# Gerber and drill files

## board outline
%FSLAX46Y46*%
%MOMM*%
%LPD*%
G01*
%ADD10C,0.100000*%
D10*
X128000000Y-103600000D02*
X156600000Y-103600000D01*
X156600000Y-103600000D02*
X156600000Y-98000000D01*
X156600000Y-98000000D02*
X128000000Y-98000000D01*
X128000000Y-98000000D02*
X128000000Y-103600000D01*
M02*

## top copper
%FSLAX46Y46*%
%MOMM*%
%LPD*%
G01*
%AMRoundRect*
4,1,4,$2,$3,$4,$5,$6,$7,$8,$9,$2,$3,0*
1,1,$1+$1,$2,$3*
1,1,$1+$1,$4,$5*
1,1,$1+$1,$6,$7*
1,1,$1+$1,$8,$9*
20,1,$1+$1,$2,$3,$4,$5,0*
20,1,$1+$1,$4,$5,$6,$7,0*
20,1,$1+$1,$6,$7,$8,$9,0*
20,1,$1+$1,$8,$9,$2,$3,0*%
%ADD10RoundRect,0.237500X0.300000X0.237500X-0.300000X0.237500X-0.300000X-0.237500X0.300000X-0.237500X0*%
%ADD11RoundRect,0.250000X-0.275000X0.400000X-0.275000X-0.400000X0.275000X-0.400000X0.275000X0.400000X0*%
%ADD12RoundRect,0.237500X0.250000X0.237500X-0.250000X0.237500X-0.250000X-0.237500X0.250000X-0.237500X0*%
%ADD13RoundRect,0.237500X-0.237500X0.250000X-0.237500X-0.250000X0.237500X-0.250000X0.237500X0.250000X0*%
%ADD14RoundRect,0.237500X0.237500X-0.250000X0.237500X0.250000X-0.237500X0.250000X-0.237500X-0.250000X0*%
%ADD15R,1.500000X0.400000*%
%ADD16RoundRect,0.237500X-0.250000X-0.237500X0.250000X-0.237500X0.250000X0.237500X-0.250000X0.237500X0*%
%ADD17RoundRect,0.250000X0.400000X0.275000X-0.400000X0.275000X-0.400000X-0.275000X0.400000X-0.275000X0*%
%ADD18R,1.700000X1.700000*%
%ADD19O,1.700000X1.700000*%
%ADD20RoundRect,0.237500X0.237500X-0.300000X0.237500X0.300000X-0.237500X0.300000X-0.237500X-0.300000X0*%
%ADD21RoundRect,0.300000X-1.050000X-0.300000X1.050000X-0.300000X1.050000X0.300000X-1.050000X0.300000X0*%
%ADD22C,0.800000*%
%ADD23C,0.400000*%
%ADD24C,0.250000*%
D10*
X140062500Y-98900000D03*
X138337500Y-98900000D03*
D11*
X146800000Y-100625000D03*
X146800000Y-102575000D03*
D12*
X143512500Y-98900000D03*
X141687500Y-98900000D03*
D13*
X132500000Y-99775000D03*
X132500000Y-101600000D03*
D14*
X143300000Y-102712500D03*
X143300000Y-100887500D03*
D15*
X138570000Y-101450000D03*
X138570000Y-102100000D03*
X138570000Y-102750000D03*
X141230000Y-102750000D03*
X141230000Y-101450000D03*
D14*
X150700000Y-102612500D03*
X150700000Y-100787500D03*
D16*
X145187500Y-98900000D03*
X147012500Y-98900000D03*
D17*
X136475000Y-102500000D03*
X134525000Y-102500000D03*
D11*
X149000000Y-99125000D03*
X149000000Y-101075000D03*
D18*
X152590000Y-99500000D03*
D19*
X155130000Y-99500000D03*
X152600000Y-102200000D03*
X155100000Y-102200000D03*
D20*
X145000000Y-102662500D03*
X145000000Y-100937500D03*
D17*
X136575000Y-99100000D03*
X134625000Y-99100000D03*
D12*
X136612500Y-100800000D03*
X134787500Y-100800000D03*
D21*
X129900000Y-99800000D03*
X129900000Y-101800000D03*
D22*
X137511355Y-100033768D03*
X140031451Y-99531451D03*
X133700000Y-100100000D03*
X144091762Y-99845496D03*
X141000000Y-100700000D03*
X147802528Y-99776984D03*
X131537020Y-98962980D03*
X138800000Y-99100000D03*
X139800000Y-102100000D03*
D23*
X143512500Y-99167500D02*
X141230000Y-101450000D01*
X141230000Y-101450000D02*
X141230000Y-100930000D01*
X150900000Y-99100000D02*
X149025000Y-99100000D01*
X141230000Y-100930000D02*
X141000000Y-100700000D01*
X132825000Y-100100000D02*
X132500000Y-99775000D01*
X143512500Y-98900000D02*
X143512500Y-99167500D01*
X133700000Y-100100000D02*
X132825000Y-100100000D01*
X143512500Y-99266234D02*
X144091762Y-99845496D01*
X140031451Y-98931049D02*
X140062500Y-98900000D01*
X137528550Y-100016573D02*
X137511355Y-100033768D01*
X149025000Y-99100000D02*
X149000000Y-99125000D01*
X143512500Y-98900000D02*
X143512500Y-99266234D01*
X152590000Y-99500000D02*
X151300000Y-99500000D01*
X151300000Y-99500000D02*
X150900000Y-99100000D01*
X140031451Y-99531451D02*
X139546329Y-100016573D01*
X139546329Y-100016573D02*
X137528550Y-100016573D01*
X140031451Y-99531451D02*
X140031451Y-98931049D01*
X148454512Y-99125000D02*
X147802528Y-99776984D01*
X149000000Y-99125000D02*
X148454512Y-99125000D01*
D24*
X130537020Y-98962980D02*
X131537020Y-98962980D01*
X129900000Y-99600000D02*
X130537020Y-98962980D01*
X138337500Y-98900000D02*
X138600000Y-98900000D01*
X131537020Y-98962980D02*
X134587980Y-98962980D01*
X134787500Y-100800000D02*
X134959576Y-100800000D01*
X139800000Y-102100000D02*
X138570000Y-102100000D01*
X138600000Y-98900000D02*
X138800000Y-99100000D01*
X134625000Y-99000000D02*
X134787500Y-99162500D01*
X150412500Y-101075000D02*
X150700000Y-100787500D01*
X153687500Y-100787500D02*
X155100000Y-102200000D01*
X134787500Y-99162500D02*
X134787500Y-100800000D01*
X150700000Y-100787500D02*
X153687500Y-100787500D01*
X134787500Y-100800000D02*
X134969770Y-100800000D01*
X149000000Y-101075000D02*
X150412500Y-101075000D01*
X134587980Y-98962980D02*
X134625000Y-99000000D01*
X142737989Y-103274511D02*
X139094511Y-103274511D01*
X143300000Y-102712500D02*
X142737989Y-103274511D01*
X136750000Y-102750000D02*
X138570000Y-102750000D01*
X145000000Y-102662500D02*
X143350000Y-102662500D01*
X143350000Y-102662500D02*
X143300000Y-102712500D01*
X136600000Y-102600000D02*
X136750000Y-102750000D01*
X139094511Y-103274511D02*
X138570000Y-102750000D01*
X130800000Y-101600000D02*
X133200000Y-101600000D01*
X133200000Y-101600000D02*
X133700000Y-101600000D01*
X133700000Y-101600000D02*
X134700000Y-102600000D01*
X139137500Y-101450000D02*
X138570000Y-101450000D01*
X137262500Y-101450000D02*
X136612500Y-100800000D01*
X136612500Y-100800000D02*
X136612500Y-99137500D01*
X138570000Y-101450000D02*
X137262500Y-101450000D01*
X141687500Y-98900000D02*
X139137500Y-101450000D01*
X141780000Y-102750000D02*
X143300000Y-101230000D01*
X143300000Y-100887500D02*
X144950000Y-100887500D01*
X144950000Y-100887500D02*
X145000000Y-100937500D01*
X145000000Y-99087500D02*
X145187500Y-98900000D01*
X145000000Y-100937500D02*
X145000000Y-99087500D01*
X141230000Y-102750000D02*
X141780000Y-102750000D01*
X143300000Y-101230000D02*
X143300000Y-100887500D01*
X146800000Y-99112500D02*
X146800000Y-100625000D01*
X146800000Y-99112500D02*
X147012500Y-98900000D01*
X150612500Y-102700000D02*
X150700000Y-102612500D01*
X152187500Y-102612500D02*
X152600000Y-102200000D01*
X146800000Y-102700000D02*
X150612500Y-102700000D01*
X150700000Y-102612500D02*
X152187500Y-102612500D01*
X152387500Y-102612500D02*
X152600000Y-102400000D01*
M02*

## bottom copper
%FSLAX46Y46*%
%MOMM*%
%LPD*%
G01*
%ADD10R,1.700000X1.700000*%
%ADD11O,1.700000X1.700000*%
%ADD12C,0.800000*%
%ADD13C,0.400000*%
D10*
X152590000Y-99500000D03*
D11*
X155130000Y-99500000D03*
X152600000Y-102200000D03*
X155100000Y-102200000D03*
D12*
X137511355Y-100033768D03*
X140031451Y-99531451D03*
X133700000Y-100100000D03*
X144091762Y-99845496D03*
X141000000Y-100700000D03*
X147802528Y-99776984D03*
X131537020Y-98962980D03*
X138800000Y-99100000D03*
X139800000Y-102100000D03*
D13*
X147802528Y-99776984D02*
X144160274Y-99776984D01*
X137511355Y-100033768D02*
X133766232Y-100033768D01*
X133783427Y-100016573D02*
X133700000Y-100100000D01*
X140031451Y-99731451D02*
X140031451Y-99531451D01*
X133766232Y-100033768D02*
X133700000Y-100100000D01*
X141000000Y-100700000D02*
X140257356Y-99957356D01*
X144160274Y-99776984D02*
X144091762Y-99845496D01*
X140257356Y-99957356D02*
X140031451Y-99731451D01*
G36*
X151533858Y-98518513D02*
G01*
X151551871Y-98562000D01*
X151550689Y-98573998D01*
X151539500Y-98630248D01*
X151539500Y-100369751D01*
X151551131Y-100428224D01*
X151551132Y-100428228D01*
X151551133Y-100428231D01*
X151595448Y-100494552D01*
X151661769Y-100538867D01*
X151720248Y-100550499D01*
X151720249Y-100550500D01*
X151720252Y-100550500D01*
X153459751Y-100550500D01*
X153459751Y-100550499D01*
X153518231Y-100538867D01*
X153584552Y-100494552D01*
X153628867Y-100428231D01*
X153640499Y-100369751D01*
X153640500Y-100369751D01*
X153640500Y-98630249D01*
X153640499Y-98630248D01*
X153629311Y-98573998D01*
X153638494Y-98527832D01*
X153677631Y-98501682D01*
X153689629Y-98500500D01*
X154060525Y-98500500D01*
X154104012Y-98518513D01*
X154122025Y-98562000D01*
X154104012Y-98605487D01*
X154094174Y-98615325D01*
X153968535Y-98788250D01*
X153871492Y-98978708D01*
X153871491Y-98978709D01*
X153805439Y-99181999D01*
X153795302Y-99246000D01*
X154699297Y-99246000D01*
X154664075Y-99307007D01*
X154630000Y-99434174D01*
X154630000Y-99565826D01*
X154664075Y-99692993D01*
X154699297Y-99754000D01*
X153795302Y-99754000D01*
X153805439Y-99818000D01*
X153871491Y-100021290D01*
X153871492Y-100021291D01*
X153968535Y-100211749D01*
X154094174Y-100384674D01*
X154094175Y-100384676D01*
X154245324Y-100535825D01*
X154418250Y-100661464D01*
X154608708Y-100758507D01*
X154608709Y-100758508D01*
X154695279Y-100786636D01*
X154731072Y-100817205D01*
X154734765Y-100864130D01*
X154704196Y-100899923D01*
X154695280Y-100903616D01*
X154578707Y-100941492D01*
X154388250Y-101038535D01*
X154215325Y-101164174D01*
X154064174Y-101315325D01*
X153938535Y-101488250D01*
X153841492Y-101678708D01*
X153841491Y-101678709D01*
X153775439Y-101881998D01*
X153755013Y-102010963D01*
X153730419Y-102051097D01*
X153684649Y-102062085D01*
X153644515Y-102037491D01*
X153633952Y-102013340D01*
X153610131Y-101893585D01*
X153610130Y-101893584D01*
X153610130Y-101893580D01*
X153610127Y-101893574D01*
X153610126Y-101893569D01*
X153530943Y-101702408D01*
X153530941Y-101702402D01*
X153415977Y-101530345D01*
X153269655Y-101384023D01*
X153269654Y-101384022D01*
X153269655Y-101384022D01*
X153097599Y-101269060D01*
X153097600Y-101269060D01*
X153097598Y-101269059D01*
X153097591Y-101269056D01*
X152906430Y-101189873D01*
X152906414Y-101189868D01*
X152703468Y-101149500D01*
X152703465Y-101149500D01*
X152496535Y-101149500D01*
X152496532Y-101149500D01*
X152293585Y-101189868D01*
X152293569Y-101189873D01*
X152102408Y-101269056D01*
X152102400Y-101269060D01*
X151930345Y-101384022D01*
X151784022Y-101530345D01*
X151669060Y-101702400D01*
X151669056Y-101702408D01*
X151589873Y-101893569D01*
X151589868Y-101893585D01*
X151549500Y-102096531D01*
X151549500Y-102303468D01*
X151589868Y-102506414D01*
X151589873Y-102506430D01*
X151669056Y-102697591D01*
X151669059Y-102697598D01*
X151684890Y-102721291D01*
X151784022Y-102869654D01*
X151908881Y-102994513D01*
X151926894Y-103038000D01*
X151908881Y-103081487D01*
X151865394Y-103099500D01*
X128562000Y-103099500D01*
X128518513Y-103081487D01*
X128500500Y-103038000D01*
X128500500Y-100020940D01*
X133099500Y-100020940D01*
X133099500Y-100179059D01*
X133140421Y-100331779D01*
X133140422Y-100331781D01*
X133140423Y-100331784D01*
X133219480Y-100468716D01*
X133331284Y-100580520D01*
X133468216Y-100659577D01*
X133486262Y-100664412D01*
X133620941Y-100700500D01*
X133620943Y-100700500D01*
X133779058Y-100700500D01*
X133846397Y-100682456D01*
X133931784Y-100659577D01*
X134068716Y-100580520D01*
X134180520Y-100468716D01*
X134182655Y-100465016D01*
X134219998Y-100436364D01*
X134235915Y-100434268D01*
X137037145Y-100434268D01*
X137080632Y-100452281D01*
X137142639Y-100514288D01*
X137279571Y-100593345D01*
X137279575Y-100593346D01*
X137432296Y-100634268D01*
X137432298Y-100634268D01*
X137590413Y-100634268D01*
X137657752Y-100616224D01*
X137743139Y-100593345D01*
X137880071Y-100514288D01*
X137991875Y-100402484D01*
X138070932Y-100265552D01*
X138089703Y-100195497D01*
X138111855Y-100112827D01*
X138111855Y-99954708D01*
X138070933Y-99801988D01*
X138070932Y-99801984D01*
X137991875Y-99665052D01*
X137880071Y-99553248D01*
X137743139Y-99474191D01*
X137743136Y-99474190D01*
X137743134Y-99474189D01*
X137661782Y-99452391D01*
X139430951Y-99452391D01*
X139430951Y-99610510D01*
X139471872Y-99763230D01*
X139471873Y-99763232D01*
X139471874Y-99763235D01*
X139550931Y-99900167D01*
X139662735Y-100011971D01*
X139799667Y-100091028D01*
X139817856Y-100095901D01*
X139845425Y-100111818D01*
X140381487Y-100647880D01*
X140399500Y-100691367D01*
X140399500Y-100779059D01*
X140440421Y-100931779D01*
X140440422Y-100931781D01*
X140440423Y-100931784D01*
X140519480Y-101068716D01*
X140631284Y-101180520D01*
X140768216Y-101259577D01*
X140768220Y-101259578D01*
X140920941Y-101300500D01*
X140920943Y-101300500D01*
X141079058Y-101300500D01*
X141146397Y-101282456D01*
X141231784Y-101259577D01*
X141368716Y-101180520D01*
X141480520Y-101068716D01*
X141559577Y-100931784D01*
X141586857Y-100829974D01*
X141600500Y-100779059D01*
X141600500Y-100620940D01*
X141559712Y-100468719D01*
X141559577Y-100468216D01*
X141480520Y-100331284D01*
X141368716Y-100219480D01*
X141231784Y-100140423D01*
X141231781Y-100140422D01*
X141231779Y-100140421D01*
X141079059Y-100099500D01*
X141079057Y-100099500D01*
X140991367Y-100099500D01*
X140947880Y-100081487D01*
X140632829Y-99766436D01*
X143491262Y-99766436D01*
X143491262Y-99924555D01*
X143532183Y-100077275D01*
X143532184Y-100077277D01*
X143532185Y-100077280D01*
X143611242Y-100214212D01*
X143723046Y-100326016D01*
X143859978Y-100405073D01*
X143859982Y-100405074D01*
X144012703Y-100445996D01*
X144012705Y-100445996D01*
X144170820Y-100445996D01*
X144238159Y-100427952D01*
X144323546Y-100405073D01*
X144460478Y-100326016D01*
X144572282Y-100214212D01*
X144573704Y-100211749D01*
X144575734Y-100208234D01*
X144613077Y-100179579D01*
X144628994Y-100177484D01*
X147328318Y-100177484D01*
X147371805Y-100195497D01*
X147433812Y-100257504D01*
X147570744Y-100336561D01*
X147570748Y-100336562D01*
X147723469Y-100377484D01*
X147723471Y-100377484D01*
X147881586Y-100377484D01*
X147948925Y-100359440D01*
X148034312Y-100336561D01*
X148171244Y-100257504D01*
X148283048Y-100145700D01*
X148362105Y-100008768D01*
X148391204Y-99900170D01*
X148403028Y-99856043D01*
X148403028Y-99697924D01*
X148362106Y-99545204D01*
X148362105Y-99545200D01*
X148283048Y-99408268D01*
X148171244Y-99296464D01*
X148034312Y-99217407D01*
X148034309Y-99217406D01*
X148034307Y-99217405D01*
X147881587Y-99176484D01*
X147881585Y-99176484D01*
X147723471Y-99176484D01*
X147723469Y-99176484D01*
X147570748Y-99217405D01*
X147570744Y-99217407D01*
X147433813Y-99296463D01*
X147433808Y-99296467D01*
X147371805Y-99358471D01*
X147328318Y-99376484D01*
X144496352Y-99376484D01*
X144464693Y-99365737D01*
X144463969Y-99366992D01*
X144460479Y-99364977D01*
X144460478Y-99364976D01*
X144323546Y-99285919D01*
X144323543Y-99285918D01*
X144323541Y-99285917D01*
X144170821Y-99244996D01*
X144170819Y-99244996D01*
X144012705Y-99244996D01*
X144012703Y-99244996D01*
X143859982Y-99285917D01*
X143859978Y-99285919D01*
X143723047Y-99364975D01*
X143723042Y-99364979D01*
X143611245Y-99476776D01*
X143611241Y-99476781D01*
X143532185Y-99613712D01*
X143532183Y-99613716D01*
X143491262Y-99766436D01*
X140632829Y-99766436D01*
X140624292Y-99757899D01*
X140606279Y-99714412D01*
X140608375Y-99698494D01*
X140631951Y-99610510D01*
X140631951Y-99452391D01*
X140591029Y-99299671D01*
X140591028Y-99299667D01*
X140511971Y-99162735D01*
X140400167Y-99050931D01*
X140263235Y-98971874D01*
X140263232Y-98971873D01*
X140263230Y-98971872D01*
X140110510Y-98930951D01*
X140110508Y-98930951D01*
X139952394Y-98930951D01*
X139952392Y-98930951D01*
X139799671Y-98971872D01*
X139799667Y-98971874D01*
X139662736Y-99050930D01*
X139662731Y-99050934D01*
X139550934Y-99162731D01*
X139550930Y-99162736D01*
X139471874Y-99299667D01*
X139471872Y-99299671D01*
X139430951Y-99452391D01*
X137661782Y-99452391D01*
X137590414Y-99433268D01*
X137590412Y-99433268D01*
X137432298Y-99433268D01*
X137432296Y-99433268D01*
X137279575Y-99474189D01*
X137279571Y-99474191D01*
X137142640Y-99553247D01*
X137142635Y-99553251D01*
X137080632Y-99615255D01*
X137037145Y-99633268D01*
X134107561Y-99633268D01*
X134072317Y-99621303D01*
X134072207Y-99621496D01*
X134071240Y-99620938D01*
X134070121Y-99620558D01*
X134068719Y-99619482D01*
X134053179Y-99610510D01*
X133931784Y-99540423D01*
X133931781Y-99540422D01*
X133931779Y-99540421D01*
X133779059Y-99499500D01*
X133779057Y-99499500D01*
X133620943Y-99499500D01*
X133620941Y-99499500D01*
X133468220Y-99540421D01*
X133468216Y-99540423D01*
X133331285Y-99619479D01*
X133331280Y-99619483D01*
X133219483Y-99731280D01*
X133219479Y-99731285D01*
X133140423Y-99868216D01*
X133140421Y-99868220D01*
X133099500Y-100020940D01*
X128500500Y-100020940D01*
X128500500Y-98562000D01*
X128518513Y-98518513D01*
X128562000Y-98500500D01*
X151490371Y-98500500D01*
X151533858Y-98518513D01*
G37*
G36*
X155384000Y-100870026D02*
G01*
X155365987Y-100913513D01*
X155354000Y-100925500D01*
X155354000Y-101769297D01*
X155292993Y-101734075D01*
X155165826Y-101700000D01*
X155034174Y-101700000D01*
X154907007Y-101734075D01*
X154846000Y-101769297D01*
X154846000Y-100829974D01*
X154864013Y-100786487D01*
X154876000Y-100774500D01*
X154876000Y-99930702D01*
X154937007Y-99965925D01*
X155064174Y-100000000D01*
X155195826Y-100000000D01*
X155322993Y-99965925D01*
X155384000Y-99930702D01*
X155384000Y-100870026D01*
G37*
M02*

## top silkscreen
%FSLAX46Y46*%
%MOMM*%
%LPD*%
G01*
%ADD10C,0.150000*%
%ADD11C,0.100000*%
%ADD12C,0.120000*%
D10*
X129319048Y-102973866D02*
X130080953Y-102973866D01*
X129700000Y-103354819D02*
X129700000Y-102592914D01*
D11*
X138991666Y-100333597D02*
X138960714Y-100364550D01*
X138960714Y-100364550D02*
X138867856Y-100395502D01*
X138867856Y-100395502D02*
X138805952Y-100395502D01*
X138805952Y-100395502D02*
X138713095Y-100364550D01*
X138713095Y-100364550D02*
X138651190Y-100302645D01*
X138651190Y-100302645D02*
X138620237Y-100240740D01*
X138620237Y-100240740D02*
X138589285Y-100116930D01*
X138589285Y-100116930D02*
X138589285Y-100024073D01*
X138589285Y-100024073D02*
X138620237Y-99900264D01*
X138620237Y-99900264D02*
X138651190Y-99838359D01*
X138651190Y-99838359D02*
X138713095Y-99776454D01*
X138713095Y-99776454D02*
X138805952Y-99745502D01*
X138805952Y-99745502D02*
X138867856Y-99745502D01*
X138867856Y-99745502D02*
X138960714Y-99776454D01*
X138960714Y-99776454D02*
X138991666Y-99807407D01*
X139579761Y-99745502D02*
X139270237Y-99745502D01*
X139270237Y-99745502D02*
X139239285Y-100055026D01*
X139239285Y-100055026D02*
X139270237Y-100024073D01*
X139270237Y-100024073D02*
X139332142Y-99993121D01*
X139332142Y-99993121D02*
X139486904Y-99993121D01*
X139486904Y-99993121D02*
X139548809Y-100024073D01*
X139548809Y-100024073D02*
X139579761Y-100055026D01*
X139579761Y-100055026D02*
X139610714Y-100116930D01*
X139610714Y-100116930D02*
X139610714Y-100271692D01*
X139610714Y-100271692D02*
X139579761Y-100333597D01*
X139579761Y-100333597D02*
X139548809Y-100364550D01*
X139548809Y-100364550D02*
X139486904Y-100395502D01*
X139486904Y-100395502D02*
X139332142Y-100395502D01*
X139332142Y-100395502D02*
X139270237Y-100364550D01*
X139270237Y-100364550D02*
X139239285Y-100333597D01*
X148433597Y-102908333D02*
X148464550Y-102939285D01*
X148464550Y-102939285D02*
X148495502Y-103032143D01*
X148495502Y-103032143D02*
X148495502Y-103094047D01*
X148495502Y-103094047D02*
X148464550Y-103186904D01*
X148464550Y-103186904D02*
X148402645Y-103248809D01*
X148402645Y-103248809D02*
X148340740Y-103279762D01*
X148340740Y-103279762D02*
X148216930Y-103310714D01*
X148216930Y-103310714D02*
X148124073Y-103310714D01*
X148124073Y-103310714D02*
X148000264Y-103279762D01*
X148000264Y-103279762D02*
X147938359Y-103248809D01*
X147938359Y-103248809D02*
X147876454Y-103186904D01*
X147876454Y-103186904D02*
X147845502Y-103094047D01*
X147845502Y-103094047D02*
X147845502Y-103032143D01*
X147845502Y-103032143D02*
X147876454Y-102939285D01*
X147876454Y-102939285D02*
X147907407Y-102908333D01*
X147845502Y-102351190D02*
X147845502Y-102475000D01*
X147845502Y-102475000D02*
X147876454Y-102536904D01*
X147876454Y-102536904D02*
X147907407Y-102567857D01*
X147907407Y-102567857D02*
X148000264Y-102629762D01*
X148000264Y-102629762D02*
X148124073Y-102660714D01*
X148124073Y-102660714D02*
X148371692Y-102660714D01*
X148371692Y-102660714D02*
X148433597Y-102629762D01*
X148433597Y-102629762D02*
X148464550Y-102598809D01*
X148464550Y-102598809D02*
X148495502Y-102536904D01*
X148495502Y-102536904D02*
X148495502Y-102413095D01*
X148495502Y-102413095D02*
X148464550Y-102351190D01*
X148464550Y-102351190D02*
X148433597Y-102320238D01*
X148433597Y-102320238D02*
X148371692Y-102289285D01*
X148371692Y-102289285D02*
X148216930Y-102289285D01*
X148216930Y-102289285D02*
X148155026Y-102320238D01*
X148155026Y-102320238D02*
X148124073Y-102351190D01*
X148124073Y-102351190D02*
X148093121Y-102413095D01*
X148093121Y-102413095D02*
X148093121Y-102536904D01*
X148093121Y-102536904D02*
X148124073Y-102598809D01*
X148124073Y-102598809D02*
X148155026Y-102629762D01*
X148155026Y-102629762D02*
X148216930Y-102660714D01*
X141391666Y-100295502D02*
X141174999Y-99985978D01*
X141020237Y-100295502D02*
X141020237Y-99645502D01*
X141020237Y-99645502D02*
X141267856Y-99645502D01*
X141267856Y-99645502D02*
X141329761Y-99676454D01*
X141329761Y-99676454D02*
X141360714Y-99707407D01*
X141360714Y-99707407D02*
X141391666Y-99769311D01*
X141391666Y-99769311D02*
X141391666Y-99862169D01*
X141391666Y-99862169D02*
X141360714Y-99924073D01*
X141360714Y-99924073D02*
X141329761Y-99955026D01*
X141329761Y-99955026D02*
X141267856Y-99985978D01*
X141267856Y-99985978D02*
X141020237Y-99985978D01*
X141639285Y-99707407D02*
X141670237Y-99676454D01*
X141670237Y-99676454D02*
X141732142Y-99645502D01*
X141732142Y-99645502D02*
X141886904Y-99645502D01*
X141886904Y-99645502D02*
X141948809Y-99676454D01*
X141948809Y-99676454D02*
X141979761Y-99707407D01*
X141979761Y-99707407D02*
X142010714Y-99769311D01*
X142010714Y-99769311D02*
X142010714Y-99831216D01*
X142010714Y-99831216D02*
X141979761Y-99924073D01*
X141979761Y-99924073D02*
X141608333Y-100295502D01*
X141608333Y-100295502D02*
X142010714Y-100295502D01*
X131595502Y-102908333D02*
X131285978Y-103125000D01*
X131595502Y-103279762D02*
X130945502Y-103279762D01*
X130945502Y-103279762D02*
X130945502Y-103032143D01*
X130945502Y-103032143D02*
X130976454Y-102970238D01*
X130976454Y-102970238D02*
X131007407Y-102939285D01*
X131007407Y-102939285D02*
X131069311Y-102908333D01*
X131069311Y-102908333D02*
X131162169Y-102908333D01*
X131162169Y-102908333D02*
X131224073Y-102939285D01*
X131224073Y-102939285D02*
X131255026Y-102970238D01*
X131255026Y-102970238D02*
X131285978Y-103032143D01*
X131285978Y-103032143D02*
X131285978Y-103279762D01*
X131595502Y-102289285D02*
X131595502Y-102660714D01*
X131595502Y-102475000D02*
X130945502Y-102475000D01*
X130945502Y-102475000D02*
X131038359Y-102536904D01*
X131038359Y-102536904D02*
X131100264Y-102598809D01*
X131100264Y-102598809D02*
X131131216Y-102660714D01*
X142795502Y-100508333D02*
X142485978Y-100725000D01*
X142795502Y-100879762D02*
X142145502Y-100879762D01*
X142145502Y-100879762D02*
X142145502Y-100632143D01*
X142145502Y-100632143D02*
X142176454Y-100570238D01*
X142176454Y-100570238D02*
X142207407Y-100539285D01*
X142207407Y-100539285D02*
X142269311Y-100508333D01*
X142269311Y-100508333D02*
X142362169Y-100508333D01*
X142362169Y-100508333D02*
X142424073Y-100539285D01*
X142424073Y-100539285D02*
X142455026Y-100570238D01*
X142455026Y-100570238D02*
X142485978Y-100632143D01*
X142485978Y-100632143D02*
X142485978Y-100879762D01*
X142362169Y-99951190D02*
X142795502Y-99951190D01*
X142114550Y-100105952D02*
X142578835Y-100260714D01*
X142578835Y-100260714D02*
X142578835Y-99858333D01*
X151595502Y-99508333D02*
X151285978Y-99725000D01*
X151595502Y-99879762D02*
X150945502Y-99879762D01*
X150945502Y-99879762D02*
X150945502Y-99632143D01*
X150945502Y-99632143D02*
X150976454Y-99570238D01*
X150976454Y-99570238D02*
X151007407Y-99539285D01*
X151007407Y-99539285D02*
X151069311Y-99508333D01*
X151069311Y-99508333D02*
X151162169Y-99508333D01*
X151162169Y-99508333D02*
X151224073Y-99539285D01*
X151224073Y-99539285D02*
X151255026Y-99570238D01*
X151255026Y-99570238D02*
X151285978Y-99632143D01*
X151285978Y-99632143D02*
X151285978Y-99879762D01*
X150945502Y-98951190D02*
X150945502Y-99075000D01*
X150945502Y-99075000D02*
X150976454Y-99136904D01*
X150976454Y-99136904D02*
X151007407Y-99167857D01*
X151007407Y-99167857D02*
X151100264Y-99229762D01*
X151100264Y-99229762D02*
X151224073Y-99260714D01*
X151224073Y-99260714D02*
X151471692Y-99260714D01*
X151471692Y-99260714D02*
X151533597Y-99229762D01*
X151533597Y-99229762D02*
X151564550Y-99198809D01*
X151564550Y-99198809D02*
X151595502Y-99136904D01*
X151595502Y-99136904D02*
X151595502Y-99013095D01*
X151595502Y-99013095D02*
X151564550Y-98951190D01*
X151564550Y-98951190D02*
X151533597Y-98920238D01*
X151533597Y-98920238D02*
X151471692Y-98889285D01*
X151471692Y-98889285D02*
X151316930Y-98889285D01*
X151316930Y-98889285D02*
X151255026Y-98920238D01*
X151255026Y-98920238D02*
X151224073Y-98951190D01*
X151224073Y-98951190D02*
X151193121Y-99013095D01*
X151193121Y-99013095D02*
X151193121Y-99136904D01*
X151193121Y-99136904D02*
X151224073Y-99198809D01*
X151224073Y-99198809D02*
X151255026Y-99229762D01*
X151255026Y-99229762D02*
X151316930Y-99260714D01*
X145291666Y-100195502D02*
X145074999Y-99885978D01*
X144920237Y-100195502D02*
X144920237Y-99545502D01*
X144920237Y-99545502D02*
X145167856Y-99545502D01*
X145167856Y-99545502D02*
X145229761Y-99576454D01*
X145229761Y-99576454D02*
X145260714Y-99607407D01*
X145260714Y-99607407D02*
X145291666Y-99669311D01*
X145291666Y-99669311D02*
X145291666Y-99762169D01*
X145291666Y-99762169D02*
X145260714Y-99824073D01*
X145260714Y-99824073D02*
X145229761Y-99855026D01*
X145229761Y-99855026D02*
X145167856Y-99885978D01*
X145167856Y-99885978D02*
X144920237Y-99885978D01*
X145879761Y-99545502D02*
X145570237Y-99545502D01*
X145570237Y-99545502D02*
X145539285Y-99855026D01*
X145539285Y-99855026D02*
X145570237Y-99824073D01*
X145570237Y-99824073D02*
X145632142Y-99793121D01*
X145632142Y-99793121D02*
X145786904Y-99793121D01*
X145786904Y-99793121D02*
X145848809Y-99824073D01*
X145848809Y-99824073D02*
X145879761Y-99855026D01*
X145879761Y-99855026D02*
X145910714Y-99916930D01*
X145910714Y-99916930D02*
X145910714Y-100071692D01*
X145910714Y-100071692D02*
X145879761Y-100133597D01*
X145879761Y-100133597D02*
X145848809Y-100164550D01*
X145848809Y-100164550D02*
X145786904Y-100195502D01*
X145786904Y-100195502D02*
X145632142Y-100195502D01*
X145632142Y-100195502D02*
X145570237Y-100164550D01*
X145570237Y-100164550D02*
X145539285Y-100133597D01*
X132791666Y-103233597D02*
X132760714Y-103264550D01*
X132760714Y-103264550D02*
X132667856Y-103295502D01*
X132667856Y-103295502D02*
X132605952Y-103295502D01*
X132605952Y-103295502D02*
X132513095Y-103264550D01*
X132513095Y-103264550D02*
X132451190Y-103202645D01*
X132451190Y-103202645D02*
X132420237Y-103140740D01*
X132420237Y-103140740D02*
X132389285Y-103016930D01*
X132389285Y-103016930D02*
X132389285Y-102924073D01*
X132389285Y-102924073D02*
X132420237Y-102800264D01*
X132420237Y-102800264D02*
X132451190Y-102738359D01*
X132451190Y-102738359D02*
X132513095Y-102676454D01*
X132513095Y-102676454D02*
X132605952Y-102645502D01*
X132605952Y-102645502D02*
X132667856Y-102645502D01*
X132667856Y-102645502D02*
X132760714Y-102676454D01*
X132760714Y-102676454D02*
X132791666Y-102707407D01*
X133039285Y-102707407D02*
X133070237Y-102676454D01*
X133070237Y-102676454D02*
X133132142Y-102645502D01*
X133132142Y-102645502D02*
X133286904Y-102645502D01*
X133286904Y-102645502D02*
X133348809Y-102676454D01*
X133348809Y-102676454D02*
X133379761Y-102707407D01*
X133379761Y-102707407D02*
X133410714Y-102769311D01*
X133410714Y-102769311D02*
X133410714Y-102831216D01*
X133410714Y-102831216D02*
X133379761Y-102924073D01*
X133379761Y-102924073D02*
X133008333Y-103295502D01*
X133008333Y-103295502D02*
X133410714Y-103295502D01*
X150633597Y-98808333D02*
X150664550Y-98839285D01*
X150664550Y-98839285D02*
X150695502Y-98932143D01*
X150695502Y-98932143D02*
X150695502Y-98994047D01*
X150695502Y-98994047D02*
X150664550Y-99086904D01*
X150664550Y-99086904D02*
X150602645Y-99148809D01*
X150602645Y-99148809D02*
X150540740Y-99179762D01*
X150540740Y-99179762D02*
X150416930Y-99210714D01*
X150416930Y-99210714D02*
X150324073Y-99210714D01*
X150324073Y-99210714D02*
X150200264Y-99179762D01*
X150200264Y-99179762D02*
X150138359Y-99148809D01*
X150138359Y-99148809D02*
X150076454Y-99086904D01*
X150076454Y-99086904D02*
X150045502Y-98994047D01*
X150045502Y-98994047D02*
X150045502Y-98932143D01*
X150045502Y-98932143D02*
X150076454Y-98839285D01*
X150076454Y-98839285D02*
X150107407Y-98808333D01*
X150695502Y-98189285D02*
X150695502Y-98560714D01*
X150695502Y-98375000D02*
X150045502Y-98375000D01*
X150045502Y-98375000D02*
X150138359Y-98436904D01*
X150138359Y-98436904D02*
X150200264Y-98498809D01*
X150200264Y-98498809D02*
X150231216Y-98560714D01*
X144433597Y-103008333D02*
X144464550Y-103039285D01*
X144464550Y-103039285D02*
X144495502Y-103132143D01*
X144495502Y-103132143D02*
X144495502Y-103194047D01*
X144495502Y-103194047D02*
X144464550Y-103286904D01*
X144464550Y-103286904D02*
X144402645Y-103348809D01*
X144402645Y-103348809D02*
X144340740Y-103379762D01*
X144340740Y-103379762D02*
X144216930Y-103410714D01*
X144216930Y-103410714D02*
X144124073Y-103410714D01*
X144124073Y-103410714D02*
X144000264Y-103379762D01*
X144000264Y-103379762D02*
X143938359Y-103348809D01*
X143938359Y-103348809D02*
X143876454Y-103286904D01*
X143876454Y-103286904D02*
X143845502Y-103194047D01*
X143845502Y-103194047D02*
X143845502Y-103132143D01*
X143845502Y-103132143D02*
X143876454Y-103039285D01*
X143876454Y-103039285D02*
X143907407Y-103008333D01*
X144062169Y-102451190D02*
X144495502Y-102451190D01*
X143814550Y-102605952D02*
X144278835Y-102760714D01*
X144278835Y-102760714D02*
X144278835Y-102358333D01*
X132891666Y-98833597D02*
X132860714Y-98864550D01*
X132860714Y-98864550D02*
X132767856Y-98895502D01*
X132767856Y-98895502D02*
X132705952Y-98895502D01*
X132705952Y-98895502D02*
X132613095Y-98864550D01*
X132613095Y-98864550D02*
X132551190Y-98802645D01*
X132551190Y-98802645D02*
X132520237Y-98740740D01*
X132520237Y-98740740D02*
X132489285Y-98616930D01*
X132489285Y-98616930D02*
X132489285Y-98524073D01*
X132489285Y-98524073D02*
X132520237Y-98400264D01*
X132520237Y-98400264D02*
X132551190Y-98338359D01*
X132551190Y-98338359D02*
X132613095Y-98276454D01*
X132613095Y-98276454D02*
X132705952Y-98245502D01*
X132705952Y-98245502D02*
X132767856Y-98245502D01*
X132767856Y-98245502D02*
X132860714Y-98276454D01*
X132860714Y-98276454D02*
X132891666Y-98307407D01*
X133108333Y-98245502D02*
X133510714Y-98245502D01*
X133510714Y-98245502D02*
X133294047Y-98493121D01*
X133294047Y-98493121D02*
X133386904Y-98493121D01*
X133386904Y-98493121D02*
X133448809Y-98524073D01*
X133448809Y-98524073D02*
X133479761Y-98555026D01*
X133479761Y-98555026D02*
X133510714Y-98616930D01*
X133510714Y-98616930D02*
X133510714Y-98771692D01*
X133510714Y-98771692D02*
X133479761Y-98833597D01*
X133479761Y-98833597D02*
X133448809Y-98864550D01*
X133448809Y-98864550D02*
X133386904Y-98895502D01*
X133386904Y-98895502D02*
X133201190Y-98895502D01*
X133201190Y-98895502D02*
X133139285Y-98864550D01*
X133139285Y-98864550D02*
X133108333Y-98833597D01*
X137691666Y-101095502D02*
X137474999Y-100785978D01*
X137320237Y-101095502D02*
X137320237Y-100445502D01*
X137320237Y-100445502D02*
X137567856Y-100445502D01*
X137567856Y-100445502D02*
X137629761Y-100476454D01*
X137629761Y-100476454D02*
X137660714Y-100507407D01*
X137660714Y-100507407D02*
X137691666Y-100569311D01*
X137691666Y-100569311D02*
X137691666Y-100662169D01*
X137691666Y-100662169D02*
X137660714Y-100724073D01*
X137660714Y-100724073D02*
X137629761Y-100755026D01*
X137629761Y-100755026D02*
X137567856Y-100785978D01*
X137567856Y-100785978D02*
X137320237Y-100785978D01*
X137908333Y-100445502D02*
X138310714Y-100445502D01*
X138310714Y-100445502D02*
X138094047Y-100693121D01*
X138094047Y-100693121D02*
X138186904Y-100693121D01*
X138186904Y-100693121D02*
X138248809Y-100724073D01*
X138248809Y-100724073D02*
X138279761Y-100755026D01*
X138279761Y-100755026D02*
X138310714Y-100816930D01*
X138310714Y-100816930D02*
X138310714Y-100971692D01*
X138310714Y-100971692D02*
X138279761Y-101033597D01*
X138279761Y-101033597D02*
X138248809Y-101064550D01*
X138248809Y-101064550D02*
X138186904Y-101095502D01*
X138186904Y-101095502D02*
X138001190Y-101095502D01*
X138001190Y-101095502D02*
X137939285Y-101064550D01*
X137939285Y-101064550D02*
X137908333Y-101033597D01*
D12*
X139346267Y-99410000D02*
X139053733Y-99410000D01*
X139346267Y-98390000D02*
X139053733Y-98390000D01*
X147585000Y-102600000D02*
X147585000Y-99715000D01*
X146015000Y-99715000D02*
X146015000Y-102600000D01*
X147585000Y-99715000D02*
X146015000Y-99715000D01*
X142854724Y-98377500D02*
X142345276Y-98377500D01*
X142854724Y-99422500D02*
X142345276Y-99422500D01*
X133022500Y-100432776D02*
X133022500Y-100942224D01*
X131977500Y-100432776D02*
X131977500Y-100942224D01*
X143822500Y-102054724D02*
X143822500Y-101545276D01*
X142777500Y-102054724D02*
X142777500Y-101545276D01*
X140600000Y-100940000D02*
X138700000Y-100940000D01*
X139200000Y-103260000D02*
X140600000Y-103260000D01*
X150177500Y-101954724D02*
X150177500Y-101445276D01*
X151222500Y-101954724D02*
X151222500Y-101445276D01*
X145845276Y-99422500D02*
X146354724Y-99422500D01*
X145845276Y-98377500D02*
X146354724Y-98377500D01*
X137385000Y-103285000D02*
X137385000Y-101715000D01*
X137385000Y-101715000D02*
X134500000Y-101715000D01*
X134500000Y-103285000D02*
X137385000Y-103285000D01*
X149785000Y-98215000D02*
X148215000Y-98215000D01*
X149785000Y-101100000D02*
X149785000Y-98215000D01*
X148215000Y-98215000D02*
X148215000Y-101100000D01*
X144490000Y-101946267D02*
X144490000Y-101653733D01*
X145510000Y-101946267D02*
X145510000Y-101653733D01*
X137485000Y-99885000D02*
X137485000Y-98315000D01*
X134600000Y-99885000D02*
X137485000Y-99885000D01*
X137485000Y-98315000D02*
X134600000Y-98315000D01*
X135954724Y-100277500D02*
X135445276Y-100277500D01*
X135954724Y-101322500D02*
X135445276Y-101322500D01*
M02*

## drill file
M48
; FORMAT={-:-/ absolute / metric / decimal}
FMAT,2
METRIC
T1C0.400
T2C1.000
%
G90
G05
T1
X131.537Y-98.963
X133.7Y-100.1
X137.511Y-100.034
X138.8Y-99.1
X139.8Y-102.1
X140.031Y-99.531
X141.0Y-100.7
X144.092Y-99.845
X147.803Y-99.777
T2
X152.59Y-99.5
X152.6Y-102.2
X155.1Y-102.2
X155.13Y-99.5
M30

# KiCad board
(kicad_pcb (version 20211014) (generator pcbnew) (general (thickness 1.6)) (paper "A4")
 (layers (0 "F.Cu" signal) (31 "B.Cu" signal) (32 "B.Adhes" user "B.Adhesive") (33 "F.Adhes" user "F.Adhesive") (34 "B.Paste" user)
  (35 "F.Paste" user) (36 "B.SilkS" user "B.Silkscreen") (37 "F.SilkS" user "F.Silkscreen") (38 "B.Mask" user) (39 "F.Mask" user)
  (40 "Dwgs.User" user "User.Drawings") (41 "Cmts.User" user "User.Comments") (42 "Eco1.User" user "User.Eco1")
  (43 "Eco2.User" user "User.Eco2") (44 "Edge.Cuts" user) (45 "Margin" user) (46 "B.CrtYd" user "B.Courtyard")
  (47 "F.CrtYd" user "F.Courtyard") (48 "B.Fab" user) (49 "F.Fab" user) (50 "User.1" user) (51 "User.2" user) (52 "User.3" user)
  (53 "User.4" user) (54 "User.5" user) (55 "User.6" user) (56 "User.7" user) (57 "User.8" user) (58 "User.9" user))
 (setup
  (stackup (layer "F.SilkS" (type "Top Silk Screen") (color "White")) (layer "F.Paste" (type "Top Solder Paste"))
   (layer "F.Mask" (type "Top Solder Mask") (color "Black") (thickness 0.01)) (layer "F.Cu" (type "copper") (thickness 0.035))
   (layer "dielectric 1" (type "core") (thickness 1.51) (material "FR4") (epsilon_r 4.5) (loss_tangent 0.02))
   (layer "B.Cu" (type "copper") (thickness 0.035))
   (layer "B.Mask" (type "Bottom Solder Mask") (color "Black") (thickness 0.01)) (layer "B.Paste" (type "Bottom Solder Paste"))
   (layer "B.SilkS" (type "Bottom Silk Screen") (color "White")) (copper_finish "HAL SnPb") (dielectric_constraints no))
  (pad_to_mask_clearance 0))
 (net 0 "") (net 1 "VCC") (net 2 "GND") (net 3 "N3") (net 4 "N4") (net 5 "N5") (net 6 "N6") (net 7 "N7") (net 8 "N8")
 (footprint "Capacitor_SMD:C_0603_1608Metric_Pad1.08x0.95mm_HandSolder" (layer "F.Cu") (at 139.2 98.9 180)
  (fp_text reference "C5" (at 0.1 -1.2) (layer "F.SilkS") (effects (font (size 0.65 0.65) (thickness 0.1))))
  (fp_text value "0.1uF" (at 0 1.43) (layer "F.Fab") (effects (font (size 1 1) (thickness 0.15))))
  (fp_line (start -0.146267 -0.51) (end 0.146267 -0.51) (layer "F.SilkS") (width 0.12))
  (fp_line (start -0.146267 0.51) (end 0.146267 0.51) (layer "F.SilkS") (width 0.12))
  (pad "1" smd roundrect locked (at -0.8625 0 180) (size 1.075 0.95) (layers "F.Cu" "F.Paste" "F.Mask") (roundrect_rratio 0.25)
   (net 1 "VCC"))
  (pad "2" smd roundrect locked (at 0.8625 0 180) (size 1.075 0.95) (layers "F.Cu" "F.Paste" "F.Mask") (roundrect_rratio 0.25) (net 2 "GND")))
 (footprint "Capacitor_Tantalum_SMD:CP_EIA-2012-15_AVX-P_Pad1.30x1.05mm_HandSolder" (layer "F.Cu") (at 146.8 101.6 -90)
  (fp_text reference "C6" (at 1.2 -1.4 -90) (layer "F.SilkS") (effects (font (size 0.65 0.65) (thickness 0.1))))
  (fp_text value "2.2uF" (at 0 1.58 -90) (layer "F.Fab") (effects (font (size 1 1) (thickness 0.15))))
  (fp_line (start 1 -0.785) (end -1.885 -0.785) (layer "F.SilkS") (width 0.12))
  (fp_line (start -1.885 0.785) (end 1 0.785) (layer "F.SilkS") (width 0.12))
  (fp_line (start -1.885 -0.785) (end -1.885 0.785) (layer "F.SilkS") (width 0.12))
  (pad "1" smd roundrect locked (at -0.975 0 270) (size 1.3 1.05) (layers "F.Cu" "F.Paste" "F.Mask") (roundrect_rratio 0.2380952381)
   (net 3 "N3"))
  (pad "2" smd roundrect locked (at 0.975 0 270) (size 1.3 1.05) (layers "F.Cu" "F.Paste" "F.Mask") (roundrect_rratio 0.2380952381)
   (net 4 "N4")))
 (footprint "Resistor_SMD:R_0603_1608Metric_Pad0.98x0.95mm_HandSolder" (layer "F.Cu") (at 142.6 98.9 180)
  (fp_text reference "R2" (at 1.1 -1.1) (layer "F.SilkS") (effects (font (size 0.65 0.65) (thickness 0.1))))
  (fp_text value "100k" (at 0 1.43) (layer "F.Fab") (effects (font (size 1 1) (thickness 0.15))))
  (fp_line (start -0.254724 0.5225) (end 0.254724 0.5225) (layer "F.SilkS") (width 0.12))
  (fp_line (start -0.254724 -0.5225) (end 0.254724 -0.5225) (layer "F.SilkS") (width 0.12))
  (pad "1" smd roundrect locked (at -0.9125 0 180) (size 0.975 0.95) (layers "F.Cu" "F.Paste" "F.Mask") (roundrect_rratio 0.25)
   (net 1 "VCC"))
  (pad "2" smd roundrect locked (at 0.9125 0 180) (size 0.975 0.95) (layers "F.Cu" "F.Paste" "F.Mask") (roundrect_rratio 0.25) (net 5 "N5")))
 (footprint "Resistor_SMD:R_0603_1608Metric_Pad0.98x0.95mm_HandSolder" (layer "F.Cu") (at 132.5 100.6875 -90)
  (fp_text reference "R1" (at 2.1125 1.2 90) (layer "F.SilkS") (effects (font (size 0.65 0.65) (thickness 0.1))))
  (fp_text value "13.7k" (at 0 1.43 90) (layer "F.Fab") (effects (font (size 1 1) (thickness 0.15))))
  (fp_line (start -0.254724 -0.5225) (end 0.254724 -0.5225) (layer "F.SilkS") (width 0.12))
  (fp_line (start -0.254724 0.5225) (end 0.254724 0.5225) (layer "F.SilkS") (width 0.12))
  (pad "1" smd roundrect locked (at -0.9125 0 270) (size 0.975 0.95) (layers "F.Cu" "F.Paste" "F.Mask") (roundrect_rratio 0.25)
   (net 1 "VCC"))
  (pad "2" smd roundrect locked (at 0.9125 0 270) (size 0.975 0.95) (layers "F.Cu" "F.Paste" "F.Mask") (roundrect_rratio 0.25) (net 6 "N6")))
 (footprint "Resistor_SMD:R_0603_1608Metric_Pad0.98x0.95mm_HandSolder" (layer "F.Cu") (at 143.3 101.8 90)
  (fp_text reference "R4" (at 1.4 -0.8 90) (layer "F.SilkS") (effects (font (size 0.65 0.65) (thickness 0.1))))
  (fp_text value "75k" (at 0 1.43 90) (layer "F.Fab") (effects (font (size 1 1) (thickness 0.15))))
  (fp_line (start -0.254724 0.5225) (end 0.254724 0.5225) (layer "F.SilkS") (width 0.12))
  (fp_line (start -0.254724 -0.5225) (end 0.254724 -0.5225) (layer "F.SilkS") (width 0.12))
  (pad "1" smd roundrect locked (at -0.9125 0 90) (size 0.975 0.95) (layers "F.Cu" "F.Paste" "F.Mask") (roundrect_rratio 0.25) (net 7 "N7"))
  (pad "2" smd roundrect locked (at 0.9125 0 90) (size 0.975 0.95) (layers "F.Cu" "F.Paste" "F.Mask") (roundrect_rratio 0.25) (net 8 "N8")))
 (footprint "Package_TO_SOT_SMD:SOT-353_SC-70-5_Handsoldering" (layer "F.Cu") (at 139.9 102.1)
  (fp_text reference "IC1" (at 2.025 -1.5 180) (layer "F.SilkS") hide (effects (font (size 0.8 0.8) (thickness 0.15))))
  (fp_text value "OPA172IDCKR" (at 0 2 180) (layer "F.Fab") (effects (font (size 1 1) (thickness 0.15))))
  (fp_line (start 0.7 -1.16) (end -1.2 -1.16) (layer "F.SilkS") (width 0.12))
  (fp_line (start -0.7 1.16) (end 0.7 1.16) (layer "F.SilkS") (width 0.12))
  (pad "1" smd rect locked (at -1.33 -0.65) (size 1.5 0.4) (layers "F.Cu" "F.Paste" "F.Mask") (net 5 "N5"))
  (pad "2" smd rect locked (at -1.33 0) (size 1.5 0.4) (layers "F.Cu" "F.Paste" "F.Mask") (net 2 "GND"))
  (pad "3" smd rect locked (at -1.33 0.65) (size 1.5 0.4) (layers "F.Cu" "F.Paste" "F.Mask") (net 7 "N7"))
  (pad "4" smd rect locked (at 1.33 0.65) (size 1.5 0.4) (layers "F.Cu" "F.Paste" "F.Mask") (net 8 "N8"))
  (pad "5" smd rect locked (at 1.33 -0.65) (size 1.5 0.4) (layers "F.Cu" "F.Paste" "F.Mask") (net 1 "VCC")))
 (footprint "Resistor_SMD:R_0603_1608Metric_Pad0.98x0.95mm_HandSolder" (layer "F.Cu") (at 150.7 101.7 90)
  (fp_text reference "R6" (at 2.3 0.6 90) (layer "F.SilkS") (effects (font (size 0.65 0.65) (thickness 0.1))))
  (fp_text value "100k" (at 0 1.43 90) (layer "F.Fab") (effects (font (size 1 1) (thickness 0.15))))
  (fp_line (start -0.254724 -0.5225) (end 0.254724 -0.5225) (layer "F.SilkS") (width 0.12))
  (fp_line (start -0.254724 0.5225) (end 0.254724 0.5225) (layer "F.SilkS") (width 0.12))
  (pad "1" smd roundrect locked (at -0.9125 0 90) (size 0.975 0.95) (layers "F.Cu" "F.Paste" "F.Mask") (roundrect_rratio 0.25) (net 4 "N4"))
  (pad "2" smd roundrect locked (at 0.9125 0 90) (size 0.975 0.95) (layers "F.Cu" "F.Paste" "F.Mask") (roundrect_rratio 0.25) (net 2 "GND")))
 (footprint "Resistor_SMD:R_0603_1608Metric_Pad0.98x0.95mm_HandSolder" (layer "F.Cu") (at 146.1 98.9)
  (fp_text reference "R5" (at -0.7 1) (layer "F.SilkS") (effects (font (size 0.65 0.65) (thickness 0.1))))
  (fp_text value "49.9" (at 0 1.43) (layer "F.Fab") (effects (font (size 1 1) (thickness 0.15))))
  (fp_line (start -0.254724 0.5225) (end 0.254724 0.5225) (layer "F.SilkS") (width 0.12))
  (fp_line (start -0.254724 -0.5225) (end 0.254724 -0.5225) (layer "F.SilkS") (width 0.12))
  (pad "1" smd roundrect locked (at -0.9125 0) (size 0.975 0.95) (layers "F.Cu" "F.Paste" "F.Mask") (roundrect_rratio 0.25) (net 8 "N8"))
  (pad "2" smd roundrect locked (at 0.9125 0) (size 0.975 0.95) (layers "F.Cu" "F.Paste" "F.Mask") (roundrect_rratio 0.25) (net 3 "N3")))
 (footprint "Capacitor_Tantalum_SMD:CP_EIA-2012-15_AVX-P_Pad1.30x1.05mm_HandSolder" (layer "F.Cu") (at 135.5 102.5 180)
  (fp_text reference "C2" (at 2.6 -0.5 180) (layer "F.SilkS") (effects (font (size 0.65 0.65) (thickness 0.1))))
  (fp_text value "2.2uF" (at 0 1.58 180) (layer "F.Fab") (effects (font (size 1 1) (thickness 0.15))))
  (fp_line (start -1.885 -0.785) (end -1.885 0.785) (layer "F.SilkS") (width 0.12))
  (fp_line (start -1.885 0.785) (end 1 0.785) (layer "F.SilkS") (width 0.12))
  (fp_line (start 1 -0.785) (end -1.885 -0.785) (layer "F.SilkS") (width 0.12))
  (pad "1" smd roundrect locked (at -0.975 0 180) (size 1.3 1.05) (layers "F.Cu" "F.Paste" "F.Mask") (roundrect_rratio 0.2380952381)
   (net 7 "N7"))
  (pad "2" smd roundrect locked (at 0.975 0 180) (size 1.3 1.05) (layers "F.Cu" "F.Paste" "F.Mask") (roundrect_rratio 0.2380952381)
   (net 6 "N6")))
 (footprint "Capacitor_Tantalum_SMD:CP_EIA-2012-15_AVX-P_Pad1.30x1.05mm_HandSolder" (layer "F.Cu") (at 149 100.1 -90)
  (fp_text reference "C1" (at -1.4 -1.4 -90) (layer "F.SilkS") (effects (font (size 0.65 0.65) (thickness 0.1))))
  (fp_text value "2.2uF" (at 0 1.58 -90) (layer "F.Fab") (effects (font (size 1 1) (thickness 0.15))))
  (fp_line (start -1.885 -0.785) (end -1.885 0.785) (layer "F.SilkS") (width 0.12))
  (fp_line (start 1 -0.785) (end -1.885 -0.785) (layer "F.SilkS") (width 0.12))
  (fp_line (start -1.885 0.785) (end 1 0.785) (layer "F.SilkS") (width 0.12))
  (pad "1" smd roundrect locked (at -0.975 0 270) (size 1.3 1.05) (layers "F.Cu" "F.Paste" "F.Mask") (roundrect_rratio 0.2380952381)
   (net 1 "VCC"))
  (pad "2" smd roundrect locked (at 0.975 0 270) (size 1.3 1.05) (layers "F.Cu" "F.Paste" "F.Mask") (roundrect_rratio 0.2380952381)
   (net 2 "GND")))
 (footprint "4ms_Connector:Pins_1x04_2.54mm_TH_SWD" (layer "F.Cu") (at 156.4 99.5 90)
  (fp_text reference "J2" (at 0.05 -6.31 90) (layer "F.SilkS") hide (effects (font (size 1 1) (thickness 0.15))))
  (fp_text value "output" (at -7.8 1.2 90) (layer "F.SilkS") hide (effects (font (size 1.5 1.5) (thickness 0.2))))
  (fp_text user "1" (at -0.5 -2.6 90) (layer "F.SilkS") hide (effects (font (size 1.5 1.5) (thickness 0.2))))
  (pad "1" thru_hole rect (at 0 -3.81 90) (size 1.7 1.7) (drill 1) (layers *.Cu *.Mask) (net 1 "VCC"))
  (pad "2" thru_hole oval (at 0 -1.27 90) (size 1.7 1.7) (drill 1) (layers *.Cu *.Mask) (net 2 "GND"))
  (pad "3" thru_hole oval (at -2.7 -3.8 90) (size 1.7 1.7) (drill 1) (layers *.Cu *.Mask) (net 4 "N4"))
  (pad "4" thru_hole oval (at -2.7 -1.3 90) (size 1.7 1.7) (drill 1) (layers *.Cu *.Mask) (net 2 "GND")))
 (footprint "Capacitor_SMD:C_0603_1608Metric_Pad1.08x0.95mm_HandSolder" (layer "F.Cu") (at 145 101.8 90)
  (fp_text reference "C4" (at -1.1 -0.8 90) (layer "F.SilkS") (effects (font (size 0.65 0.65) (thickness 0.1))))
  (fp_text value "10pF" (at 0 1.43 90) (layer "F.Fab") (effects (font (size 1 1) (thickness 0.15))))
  (fp_line (start -0.146267 -0.51) (end 0.146267 -0.51) (layer "F.SilkS") (width 0.12))
  (fp_line (start -0.146267 0.51) (end 0.146267 0.51) (layer "F.SilkS") (width 0.12))
  (pad "1" smd roundrect locked (at -0.8625 0 90) (size 1.075 0.95) (layers "F.Cu" "F.Paste" "F.Mask") (roundrect_rratio 0.25) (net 7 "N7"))
  (pad "2" smd roundrect locked (at 0.8625 0 90) (size 1.075 0.95) (layers "F.Cu" "F.Paste" "F.Mask") (roundrect_rratio 0.25) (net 8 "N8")))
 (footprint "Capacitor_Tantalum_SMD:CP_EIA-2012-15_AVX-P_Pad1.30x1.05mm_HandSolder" (layer "F.Cu") (at 135.6 99.1 180)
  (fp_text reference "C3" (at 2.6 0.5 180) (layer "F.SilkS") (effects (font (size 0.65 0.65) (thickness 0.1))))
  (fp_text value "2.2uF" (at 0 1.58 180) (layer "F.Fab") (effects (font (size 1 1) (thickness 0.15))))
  (fp_line (start -1.885 -0.785) (end -1.885 0.785) (layer "F.SilkS") (width 0.12))
  (fp_line (start 1 -0.785) (end -1.885 -0.785) (layer "F.SilkS") (width 0.12))
  (fp_line (start -1.885 0.785) (end 1 0.785) (layer "F.SilkS") (width 0.12))
  (pad "1" smd roundrect locked (at -0.975 0 180) (size 1.3 1.05) (layers "F.Cu" "F.Paste" "F.Mask") (roundrect_rratio 0.2380952381)
   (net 5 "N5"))
  (pad "2" smd roundrect locked (at 0.975 0 180) (size 1.3 1.05) (layers "F.Cu" "F.Paste" "F.Mask") (roundrect_rratio 0.2380952381)
   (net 2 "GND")))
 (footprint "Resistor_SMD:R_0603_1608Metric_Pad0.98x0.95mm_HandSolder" (layer "F.Cu") (at 135.7 100.8 180)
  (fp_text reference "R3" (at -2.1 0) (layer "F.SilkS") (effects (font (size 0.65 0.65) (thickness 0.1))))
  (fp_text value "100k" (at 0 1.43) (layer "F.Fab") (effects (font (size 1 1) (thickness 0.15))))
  (fp_line (start -0.254724 0.5225) (end 0.254724 0.5225) (layer "F.SilkS") (width 0.12))
  (fp_line (start -0.254724 -0.5225) (end 0.254724 -0.5225) (layer "F.SilkS") (width 0.12))
  (pad "1" smd roundrect locked (at -0.9125 0 180) (size 0.975 0.95) (layers "F.Cu" "F.Paste" "F.Mask") (roundrect_rratio 0.25) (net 5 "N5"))
  (pad "2" smd roundrect locked (at 0.9125 0 180) (size 0.975 0.95) (layers "F.Cu" "F.Paste" "F.Mask") (roundrect_rratio 0.25) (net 2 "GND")))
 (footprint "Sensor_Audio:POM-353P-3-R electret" (layer "F.Cu") (at 129.9 100.8)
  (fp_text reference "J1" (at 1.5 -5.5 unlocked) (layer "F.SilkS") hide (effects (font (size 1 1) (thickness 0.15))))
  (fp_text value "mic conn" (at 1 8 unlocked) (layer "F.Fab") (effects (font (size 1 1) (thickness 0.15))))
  (pad "1" smd roundrect (at 0 -1) (size 2.7 1.2) (layers "F.Cu" "F.Paste" "F.Mask") (roundrect_rratio 0.25) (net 2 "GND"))
  (pad "2" smd roundrect (at 0 1) (size 2.7 1.2) (layers "F.Cu" "F.Paste" "F.Mask") (roundrect_rratio 0.25) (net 6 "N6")))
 (gr_line (start 128 103.6) (end 156.6 103.6) (layer "Edge.Cuts") (width 0.1))
 (gr_line (start 156.6 103.6) (end 156.6 98) (layer "Edge.Cuts") (width 0.1))
 (gr_line (start 156.6 98) (end 128 98) (layer "Edge.Cuts") (width 0.1))
 (gr_line (start 128 98) (end 128 103.6) (layer "Edge.Cuts") (width 0.1))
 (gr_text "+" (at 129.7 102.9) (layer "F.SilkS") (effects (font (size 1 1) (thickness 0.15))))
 (segment (start 143.5125 99.1675) (end 141.23 101.45) (width 0.4) (layer "F.Cu") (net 1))
 (segment (start 141.23 101.45) (end 141.23 100.93) (width 0.4) (layer "F.Cu") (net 1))
 (segment (start 150.9 99.1) (end 149.025 99.1) (width 0.4) (layer "F.Cu") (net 1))
 (segment (start 141.23 100.93) (end 141 100.7) (width 0.4) (layer "F.Cu") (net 1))
 (segment (start 132.825 100.1) (end 132.5 99.775) (width 0.4) (layer "F.Cu") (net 1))
 (segment (start 143.5125 98.9) (end 143.5125 99.1675) (width 0.4) (layer "F.Cu") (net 1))
 (segment (start 133.7 100.1) (end 132.825 100.1) (width 0.4) (layer "F.Cu") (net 1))
 (segment (start 143.5125 99.266234) (end 144.091762 99.845496) (width 0.4) (layer "F.Cu") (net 1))
 (segment (start 140.031451 98.931049) (end 140.0625 98.9) (width 0.4) (layer "F.Cu") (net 1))
 (segment (start 137.52855 100.016573) (end 137.511355 100.033768) (width 0.4) (layer "F.Cu") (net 1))
 (segment (start 149.025 99.1) (end 149 99.125) (width 0.4) (layer "F.Cu") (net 1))
 (segment (start 143.5125 98.9) (end 143.5125 99.266234) (width 0.4) (layer "F.Cu") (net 1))
 (segment (start 152.59 99.5) (end 151.3 99.5) (width 0.4) (layer "F.Cu") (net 1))
 (segment (start 151.3 99.5) (end 150.9 99.1) (width 0.4) (layer "F.Cu") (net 1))
 (segment (start 140.031451 99.531451) (end 139.546329 100.016573) (width 0.4) (layer "F.Cu") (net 1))
 (segment (start 139.546329 100.016573) (end 137.52855 100.016573) (width 0.4) (layer "F.Cu") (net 1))
 (segment (start 140.031451 99.531451) (end 140.031451 98.931049) (width 0.4) (layer "F.Cu") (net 1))
 (segment (start 148.454512 99.125) (end 147.802528 99.776984) (width 0.4) (layer "F.Cu") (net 1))
 (segment (start 149 99.125) (end 148.454512 99.125) (width 0.4) (layer "F.Cu") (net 1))
 (via (at 137.511355 100.033768) (size 0.8) (drill 0.4) (layers "F.Cu" "B.Cu") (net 1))
 (via (at 140.031451 99.531451) (size 0.8) (drill 0.4) (layers "F.Cu" "B.Cu") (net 1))
 (via (at 133.7 100.1) (size 0.8) (drill 0.4) (layers "F.Cu" "B.Cu") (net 1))
 (via (at 144.091762 99.845496) (size 0.8) (drill 0.4) (layers "F.Cu" "B.Cu") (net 1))
 (via (at 141 100.7) (size 0.8) (drill 0.4) (layers "F.Cu" "B.Cu") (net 1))
 (via (at 147.802528 99.776984) (size 0.8) (drill 0.4) (layers "F.Cu" "B.Cu") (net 1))
 (segment (start 147.802528 99.776984) (end 144.160274 99.776984) (width 0.4) (layer "B.Cu") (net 1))
 (segment (start 137.511355 100.033768) (end 133.766232 100.033768) (width 0.4) (layer "B.Cu") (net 1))
 (segment (start 133.783427 100.016573) (end 133.7 100.1) (width 0.4) (layer "B.Cu") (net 1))
 (segment (start 140.031451 99.731451) (end 140.031451 99.531451) (width 0.4) (layer "B.Cu") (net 1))
 (segment (start 133.766232 100.033768) (end 133.7 100.1) (width 0.4) (layer "B.Cu") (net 1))
 (segment (start 141 100.7) (end 140.257356 99.957356) (width 0.4) (layer "B.Cu") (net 1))
 (segment (start 144.160274 99.776984) (end 144.091762 99.845496) (width 0.4) (layer "B.Cu") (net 1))
 (segment (start 140.257356 99.957356) (end 140.031451 99.731451) (width 0.4) (layer "B.Cu") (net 1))
 (segment (start 130.53702 98.96298) (end 131.53702 98.96298) (width 0.25) (layer "F.Cu") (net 2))
 (segment (start 129.9 99.6) (end 130.53702 98.96298) (width 0.25) (layer "F.Cu") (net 2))
 (segment (start 138.3375 98.9) (end 138.6 98.9) (width 0.25) (layer "F.Cu") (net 2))
 (segment (start 131.53702 98.96298) (end 134.58798 98.96298) (width 0.25) (layer "F.Cu") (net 2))
 (segment (start 134.7875 100.8) (end 134.959576 100.8) (width 0.25) (layer "F.Cu") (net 2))
 (segment (start 139.8 102.1) (end 138.57 102.1) (width 0.25) (layer "F.Cu") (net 2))
 (segment (start 138.6 98.9) (end 138.8 99.1) (width 0.25) (layer "F.Cu") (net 2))
 (segment (start 134.625 99) (end 134.7875 99.1625) (width 0.25) (layer "F.Cu") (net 2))
 (segment (start 150.4125 101.075) (end 150.7 100.7875) (width 0.25) (layer "F.Cu") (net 2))
 (segment (start 153.6875 100.7875) (end 155.1 102.2) (width 0.25) (layer "F.Cu") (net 2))
 (segment (start 134.7875 99.1625) (end 134.7875 100.8) (width 0.25) (layer "F.Cu") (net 2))
 (segment (start 150.7 100.7875) (end 153.6875 100.7875) (width 0.25) (layer "F.Cu") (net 2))
 (segment (start 134.7875 100.8) (end 134.96977 100.8) (width 0.25) (layer "F.Cu") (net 2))
 (segment (start 149 101.075) (end 150.4125 101.075) (width 0.25) (layer "F.Cu") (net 2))
 (segment (start 134.58798 98.96298) (end 134.625 99) (width 0.25) (layer "F.Cu") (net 2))
 (via (at 131.53702 98.96298) (size 0.8) (drill 0.4) (layers "F.Cu" "B.Cu") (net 2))
 (via (at 138.8 99.1) (size 0.8) (drill 0.4) (layers "F.Cu" "B.Cu") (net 2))
 (via (at 139.8 102.1) (size 0.8) (drill 0.4) (layers "F.Cu" "B.Cu") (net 2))
 (segment (start 142.737989 103.274511) (end 139.094511 103.274511) (width 0.25) (layer "F.Cu") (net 7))
 (segment (start 143.3 102.7125) (end 142.737989 103.274511) (width 0.25) (layer "F.Cu") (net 7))
 (segment (start 136.75 102.75) (end 138.57 102.75) (width 0.25) (layer "F.Cu") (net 7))
 (segment (start 145 102.6625) (end 143.35 102.6625) (width 0.25) (layer "F.Cu") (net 7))
 (segment (start 143.35 102.6625) (end 143.3 102.7125) (width 0.25) (layer "F.Cu") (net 7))
 (segment (start 136.6 102.6) (end 136.75 102.75) (width 0.25) (layer "F.Cu") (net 7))
 (segment (start 139.094511 103.274511) (end 138.57 102.75) (width 0.25) (layer "F.Cu") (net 7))
 (segment (start 130.8 101.6) (end 133.2 101.6) (width 0.25) (layer "F.Cu") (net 6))
 (segment (start 133.2 101.6) (end 133.7 101.6) (width 0.25) (layer "F.Cu") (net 6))
 (segment (start 133.7 101.6) (end 134.7 102.6) (width 0.25) (layer "F.Cu") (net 6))
 (segment (start 139.1375 101.45) (end 138.57 101.45) (width 0.25) (layer "F.Cu") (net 5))
 (segment (start 137.2625 101.45) (end 136.6125 100.8) (width 0.25) (layer "F.Cu") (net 5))
 (segment (start 136.6125 100.8) (end 136.6125 99.1375) (width 0.25) (layer "F.Cu") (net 5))
 (segment (start 138.57 101.45) (end 137.2625 101.45) (width 0.25) (layer "F.Cu") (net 5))
 (segment (start 141.6875 98.9) (end 139.1375 101.45) (width 0.25) (layer "F.Cu") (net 5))
 (segment (start 141.78 102.75) (end 143.3 101.23) (width 0.25) (layer "F.Cu") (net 8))
 (segment (start 143.3 100.8875) (end 144.95 100.8875) (width 0.25) (layer "F.Cu") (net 8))
 (segment (start 144.95 100.8875) (end 145 100.9375) (width 0.25) (layer "F.Cu") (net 8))
 (segment (start 145 99.0875) (end 145.1875 98.9) (width 0.25) (layer "F.Cu") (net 8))
 (segment (start 145 100.9375) (end 145 99.0875) (width 0.25) (layer "F.Cu") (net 8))
 (segment (start 141.23 102.75) (end 141.78 102.75) (width 0.25) (layer "F.Cu") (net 8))
 (segment (start 143.3 101.23) (end 143.3 100.8875) (width 0.25) (layer "F.Cu") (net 8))
 (segment (start 146.8 99.1125) (end 146.8 100.625) (width 0.25) (layer "F.Cu") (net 3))
 (segment (start 146.8 99.1125) (end 147.0125 98.9) (width 0.25) (layer "F.Cu") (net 3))
 (segment (start 150.6125 102.7) (end 150.7 102.6125) (width 0.25) (layer "F.Cu") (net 4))
 (segment (start 152.1875 102.6125) (end 152.6 102.2) (width 0.25) (layer "F.Cu") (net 4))
 (segment (start 146.8 102.7) (end 150.6125 102.7) (width 0.25) (layer "F.Cu") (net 4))
 (segment (start 150.7 102.6125) (end 152.1875 102.6125) (width 0.25) (layer "F.Cu") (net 4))
 (segment (start 152.3875 102.6125) (end 152.6 102.4) (width 0.25) (layer "F.Cu") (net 4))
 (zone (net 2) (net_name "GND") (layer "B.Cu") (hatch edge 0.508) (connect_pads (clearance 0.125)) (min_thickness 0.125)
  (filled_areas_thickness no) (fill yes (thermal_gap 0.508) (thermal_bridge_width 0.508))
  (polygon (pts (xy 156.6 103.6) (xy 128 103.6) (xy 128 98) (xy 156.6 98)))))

